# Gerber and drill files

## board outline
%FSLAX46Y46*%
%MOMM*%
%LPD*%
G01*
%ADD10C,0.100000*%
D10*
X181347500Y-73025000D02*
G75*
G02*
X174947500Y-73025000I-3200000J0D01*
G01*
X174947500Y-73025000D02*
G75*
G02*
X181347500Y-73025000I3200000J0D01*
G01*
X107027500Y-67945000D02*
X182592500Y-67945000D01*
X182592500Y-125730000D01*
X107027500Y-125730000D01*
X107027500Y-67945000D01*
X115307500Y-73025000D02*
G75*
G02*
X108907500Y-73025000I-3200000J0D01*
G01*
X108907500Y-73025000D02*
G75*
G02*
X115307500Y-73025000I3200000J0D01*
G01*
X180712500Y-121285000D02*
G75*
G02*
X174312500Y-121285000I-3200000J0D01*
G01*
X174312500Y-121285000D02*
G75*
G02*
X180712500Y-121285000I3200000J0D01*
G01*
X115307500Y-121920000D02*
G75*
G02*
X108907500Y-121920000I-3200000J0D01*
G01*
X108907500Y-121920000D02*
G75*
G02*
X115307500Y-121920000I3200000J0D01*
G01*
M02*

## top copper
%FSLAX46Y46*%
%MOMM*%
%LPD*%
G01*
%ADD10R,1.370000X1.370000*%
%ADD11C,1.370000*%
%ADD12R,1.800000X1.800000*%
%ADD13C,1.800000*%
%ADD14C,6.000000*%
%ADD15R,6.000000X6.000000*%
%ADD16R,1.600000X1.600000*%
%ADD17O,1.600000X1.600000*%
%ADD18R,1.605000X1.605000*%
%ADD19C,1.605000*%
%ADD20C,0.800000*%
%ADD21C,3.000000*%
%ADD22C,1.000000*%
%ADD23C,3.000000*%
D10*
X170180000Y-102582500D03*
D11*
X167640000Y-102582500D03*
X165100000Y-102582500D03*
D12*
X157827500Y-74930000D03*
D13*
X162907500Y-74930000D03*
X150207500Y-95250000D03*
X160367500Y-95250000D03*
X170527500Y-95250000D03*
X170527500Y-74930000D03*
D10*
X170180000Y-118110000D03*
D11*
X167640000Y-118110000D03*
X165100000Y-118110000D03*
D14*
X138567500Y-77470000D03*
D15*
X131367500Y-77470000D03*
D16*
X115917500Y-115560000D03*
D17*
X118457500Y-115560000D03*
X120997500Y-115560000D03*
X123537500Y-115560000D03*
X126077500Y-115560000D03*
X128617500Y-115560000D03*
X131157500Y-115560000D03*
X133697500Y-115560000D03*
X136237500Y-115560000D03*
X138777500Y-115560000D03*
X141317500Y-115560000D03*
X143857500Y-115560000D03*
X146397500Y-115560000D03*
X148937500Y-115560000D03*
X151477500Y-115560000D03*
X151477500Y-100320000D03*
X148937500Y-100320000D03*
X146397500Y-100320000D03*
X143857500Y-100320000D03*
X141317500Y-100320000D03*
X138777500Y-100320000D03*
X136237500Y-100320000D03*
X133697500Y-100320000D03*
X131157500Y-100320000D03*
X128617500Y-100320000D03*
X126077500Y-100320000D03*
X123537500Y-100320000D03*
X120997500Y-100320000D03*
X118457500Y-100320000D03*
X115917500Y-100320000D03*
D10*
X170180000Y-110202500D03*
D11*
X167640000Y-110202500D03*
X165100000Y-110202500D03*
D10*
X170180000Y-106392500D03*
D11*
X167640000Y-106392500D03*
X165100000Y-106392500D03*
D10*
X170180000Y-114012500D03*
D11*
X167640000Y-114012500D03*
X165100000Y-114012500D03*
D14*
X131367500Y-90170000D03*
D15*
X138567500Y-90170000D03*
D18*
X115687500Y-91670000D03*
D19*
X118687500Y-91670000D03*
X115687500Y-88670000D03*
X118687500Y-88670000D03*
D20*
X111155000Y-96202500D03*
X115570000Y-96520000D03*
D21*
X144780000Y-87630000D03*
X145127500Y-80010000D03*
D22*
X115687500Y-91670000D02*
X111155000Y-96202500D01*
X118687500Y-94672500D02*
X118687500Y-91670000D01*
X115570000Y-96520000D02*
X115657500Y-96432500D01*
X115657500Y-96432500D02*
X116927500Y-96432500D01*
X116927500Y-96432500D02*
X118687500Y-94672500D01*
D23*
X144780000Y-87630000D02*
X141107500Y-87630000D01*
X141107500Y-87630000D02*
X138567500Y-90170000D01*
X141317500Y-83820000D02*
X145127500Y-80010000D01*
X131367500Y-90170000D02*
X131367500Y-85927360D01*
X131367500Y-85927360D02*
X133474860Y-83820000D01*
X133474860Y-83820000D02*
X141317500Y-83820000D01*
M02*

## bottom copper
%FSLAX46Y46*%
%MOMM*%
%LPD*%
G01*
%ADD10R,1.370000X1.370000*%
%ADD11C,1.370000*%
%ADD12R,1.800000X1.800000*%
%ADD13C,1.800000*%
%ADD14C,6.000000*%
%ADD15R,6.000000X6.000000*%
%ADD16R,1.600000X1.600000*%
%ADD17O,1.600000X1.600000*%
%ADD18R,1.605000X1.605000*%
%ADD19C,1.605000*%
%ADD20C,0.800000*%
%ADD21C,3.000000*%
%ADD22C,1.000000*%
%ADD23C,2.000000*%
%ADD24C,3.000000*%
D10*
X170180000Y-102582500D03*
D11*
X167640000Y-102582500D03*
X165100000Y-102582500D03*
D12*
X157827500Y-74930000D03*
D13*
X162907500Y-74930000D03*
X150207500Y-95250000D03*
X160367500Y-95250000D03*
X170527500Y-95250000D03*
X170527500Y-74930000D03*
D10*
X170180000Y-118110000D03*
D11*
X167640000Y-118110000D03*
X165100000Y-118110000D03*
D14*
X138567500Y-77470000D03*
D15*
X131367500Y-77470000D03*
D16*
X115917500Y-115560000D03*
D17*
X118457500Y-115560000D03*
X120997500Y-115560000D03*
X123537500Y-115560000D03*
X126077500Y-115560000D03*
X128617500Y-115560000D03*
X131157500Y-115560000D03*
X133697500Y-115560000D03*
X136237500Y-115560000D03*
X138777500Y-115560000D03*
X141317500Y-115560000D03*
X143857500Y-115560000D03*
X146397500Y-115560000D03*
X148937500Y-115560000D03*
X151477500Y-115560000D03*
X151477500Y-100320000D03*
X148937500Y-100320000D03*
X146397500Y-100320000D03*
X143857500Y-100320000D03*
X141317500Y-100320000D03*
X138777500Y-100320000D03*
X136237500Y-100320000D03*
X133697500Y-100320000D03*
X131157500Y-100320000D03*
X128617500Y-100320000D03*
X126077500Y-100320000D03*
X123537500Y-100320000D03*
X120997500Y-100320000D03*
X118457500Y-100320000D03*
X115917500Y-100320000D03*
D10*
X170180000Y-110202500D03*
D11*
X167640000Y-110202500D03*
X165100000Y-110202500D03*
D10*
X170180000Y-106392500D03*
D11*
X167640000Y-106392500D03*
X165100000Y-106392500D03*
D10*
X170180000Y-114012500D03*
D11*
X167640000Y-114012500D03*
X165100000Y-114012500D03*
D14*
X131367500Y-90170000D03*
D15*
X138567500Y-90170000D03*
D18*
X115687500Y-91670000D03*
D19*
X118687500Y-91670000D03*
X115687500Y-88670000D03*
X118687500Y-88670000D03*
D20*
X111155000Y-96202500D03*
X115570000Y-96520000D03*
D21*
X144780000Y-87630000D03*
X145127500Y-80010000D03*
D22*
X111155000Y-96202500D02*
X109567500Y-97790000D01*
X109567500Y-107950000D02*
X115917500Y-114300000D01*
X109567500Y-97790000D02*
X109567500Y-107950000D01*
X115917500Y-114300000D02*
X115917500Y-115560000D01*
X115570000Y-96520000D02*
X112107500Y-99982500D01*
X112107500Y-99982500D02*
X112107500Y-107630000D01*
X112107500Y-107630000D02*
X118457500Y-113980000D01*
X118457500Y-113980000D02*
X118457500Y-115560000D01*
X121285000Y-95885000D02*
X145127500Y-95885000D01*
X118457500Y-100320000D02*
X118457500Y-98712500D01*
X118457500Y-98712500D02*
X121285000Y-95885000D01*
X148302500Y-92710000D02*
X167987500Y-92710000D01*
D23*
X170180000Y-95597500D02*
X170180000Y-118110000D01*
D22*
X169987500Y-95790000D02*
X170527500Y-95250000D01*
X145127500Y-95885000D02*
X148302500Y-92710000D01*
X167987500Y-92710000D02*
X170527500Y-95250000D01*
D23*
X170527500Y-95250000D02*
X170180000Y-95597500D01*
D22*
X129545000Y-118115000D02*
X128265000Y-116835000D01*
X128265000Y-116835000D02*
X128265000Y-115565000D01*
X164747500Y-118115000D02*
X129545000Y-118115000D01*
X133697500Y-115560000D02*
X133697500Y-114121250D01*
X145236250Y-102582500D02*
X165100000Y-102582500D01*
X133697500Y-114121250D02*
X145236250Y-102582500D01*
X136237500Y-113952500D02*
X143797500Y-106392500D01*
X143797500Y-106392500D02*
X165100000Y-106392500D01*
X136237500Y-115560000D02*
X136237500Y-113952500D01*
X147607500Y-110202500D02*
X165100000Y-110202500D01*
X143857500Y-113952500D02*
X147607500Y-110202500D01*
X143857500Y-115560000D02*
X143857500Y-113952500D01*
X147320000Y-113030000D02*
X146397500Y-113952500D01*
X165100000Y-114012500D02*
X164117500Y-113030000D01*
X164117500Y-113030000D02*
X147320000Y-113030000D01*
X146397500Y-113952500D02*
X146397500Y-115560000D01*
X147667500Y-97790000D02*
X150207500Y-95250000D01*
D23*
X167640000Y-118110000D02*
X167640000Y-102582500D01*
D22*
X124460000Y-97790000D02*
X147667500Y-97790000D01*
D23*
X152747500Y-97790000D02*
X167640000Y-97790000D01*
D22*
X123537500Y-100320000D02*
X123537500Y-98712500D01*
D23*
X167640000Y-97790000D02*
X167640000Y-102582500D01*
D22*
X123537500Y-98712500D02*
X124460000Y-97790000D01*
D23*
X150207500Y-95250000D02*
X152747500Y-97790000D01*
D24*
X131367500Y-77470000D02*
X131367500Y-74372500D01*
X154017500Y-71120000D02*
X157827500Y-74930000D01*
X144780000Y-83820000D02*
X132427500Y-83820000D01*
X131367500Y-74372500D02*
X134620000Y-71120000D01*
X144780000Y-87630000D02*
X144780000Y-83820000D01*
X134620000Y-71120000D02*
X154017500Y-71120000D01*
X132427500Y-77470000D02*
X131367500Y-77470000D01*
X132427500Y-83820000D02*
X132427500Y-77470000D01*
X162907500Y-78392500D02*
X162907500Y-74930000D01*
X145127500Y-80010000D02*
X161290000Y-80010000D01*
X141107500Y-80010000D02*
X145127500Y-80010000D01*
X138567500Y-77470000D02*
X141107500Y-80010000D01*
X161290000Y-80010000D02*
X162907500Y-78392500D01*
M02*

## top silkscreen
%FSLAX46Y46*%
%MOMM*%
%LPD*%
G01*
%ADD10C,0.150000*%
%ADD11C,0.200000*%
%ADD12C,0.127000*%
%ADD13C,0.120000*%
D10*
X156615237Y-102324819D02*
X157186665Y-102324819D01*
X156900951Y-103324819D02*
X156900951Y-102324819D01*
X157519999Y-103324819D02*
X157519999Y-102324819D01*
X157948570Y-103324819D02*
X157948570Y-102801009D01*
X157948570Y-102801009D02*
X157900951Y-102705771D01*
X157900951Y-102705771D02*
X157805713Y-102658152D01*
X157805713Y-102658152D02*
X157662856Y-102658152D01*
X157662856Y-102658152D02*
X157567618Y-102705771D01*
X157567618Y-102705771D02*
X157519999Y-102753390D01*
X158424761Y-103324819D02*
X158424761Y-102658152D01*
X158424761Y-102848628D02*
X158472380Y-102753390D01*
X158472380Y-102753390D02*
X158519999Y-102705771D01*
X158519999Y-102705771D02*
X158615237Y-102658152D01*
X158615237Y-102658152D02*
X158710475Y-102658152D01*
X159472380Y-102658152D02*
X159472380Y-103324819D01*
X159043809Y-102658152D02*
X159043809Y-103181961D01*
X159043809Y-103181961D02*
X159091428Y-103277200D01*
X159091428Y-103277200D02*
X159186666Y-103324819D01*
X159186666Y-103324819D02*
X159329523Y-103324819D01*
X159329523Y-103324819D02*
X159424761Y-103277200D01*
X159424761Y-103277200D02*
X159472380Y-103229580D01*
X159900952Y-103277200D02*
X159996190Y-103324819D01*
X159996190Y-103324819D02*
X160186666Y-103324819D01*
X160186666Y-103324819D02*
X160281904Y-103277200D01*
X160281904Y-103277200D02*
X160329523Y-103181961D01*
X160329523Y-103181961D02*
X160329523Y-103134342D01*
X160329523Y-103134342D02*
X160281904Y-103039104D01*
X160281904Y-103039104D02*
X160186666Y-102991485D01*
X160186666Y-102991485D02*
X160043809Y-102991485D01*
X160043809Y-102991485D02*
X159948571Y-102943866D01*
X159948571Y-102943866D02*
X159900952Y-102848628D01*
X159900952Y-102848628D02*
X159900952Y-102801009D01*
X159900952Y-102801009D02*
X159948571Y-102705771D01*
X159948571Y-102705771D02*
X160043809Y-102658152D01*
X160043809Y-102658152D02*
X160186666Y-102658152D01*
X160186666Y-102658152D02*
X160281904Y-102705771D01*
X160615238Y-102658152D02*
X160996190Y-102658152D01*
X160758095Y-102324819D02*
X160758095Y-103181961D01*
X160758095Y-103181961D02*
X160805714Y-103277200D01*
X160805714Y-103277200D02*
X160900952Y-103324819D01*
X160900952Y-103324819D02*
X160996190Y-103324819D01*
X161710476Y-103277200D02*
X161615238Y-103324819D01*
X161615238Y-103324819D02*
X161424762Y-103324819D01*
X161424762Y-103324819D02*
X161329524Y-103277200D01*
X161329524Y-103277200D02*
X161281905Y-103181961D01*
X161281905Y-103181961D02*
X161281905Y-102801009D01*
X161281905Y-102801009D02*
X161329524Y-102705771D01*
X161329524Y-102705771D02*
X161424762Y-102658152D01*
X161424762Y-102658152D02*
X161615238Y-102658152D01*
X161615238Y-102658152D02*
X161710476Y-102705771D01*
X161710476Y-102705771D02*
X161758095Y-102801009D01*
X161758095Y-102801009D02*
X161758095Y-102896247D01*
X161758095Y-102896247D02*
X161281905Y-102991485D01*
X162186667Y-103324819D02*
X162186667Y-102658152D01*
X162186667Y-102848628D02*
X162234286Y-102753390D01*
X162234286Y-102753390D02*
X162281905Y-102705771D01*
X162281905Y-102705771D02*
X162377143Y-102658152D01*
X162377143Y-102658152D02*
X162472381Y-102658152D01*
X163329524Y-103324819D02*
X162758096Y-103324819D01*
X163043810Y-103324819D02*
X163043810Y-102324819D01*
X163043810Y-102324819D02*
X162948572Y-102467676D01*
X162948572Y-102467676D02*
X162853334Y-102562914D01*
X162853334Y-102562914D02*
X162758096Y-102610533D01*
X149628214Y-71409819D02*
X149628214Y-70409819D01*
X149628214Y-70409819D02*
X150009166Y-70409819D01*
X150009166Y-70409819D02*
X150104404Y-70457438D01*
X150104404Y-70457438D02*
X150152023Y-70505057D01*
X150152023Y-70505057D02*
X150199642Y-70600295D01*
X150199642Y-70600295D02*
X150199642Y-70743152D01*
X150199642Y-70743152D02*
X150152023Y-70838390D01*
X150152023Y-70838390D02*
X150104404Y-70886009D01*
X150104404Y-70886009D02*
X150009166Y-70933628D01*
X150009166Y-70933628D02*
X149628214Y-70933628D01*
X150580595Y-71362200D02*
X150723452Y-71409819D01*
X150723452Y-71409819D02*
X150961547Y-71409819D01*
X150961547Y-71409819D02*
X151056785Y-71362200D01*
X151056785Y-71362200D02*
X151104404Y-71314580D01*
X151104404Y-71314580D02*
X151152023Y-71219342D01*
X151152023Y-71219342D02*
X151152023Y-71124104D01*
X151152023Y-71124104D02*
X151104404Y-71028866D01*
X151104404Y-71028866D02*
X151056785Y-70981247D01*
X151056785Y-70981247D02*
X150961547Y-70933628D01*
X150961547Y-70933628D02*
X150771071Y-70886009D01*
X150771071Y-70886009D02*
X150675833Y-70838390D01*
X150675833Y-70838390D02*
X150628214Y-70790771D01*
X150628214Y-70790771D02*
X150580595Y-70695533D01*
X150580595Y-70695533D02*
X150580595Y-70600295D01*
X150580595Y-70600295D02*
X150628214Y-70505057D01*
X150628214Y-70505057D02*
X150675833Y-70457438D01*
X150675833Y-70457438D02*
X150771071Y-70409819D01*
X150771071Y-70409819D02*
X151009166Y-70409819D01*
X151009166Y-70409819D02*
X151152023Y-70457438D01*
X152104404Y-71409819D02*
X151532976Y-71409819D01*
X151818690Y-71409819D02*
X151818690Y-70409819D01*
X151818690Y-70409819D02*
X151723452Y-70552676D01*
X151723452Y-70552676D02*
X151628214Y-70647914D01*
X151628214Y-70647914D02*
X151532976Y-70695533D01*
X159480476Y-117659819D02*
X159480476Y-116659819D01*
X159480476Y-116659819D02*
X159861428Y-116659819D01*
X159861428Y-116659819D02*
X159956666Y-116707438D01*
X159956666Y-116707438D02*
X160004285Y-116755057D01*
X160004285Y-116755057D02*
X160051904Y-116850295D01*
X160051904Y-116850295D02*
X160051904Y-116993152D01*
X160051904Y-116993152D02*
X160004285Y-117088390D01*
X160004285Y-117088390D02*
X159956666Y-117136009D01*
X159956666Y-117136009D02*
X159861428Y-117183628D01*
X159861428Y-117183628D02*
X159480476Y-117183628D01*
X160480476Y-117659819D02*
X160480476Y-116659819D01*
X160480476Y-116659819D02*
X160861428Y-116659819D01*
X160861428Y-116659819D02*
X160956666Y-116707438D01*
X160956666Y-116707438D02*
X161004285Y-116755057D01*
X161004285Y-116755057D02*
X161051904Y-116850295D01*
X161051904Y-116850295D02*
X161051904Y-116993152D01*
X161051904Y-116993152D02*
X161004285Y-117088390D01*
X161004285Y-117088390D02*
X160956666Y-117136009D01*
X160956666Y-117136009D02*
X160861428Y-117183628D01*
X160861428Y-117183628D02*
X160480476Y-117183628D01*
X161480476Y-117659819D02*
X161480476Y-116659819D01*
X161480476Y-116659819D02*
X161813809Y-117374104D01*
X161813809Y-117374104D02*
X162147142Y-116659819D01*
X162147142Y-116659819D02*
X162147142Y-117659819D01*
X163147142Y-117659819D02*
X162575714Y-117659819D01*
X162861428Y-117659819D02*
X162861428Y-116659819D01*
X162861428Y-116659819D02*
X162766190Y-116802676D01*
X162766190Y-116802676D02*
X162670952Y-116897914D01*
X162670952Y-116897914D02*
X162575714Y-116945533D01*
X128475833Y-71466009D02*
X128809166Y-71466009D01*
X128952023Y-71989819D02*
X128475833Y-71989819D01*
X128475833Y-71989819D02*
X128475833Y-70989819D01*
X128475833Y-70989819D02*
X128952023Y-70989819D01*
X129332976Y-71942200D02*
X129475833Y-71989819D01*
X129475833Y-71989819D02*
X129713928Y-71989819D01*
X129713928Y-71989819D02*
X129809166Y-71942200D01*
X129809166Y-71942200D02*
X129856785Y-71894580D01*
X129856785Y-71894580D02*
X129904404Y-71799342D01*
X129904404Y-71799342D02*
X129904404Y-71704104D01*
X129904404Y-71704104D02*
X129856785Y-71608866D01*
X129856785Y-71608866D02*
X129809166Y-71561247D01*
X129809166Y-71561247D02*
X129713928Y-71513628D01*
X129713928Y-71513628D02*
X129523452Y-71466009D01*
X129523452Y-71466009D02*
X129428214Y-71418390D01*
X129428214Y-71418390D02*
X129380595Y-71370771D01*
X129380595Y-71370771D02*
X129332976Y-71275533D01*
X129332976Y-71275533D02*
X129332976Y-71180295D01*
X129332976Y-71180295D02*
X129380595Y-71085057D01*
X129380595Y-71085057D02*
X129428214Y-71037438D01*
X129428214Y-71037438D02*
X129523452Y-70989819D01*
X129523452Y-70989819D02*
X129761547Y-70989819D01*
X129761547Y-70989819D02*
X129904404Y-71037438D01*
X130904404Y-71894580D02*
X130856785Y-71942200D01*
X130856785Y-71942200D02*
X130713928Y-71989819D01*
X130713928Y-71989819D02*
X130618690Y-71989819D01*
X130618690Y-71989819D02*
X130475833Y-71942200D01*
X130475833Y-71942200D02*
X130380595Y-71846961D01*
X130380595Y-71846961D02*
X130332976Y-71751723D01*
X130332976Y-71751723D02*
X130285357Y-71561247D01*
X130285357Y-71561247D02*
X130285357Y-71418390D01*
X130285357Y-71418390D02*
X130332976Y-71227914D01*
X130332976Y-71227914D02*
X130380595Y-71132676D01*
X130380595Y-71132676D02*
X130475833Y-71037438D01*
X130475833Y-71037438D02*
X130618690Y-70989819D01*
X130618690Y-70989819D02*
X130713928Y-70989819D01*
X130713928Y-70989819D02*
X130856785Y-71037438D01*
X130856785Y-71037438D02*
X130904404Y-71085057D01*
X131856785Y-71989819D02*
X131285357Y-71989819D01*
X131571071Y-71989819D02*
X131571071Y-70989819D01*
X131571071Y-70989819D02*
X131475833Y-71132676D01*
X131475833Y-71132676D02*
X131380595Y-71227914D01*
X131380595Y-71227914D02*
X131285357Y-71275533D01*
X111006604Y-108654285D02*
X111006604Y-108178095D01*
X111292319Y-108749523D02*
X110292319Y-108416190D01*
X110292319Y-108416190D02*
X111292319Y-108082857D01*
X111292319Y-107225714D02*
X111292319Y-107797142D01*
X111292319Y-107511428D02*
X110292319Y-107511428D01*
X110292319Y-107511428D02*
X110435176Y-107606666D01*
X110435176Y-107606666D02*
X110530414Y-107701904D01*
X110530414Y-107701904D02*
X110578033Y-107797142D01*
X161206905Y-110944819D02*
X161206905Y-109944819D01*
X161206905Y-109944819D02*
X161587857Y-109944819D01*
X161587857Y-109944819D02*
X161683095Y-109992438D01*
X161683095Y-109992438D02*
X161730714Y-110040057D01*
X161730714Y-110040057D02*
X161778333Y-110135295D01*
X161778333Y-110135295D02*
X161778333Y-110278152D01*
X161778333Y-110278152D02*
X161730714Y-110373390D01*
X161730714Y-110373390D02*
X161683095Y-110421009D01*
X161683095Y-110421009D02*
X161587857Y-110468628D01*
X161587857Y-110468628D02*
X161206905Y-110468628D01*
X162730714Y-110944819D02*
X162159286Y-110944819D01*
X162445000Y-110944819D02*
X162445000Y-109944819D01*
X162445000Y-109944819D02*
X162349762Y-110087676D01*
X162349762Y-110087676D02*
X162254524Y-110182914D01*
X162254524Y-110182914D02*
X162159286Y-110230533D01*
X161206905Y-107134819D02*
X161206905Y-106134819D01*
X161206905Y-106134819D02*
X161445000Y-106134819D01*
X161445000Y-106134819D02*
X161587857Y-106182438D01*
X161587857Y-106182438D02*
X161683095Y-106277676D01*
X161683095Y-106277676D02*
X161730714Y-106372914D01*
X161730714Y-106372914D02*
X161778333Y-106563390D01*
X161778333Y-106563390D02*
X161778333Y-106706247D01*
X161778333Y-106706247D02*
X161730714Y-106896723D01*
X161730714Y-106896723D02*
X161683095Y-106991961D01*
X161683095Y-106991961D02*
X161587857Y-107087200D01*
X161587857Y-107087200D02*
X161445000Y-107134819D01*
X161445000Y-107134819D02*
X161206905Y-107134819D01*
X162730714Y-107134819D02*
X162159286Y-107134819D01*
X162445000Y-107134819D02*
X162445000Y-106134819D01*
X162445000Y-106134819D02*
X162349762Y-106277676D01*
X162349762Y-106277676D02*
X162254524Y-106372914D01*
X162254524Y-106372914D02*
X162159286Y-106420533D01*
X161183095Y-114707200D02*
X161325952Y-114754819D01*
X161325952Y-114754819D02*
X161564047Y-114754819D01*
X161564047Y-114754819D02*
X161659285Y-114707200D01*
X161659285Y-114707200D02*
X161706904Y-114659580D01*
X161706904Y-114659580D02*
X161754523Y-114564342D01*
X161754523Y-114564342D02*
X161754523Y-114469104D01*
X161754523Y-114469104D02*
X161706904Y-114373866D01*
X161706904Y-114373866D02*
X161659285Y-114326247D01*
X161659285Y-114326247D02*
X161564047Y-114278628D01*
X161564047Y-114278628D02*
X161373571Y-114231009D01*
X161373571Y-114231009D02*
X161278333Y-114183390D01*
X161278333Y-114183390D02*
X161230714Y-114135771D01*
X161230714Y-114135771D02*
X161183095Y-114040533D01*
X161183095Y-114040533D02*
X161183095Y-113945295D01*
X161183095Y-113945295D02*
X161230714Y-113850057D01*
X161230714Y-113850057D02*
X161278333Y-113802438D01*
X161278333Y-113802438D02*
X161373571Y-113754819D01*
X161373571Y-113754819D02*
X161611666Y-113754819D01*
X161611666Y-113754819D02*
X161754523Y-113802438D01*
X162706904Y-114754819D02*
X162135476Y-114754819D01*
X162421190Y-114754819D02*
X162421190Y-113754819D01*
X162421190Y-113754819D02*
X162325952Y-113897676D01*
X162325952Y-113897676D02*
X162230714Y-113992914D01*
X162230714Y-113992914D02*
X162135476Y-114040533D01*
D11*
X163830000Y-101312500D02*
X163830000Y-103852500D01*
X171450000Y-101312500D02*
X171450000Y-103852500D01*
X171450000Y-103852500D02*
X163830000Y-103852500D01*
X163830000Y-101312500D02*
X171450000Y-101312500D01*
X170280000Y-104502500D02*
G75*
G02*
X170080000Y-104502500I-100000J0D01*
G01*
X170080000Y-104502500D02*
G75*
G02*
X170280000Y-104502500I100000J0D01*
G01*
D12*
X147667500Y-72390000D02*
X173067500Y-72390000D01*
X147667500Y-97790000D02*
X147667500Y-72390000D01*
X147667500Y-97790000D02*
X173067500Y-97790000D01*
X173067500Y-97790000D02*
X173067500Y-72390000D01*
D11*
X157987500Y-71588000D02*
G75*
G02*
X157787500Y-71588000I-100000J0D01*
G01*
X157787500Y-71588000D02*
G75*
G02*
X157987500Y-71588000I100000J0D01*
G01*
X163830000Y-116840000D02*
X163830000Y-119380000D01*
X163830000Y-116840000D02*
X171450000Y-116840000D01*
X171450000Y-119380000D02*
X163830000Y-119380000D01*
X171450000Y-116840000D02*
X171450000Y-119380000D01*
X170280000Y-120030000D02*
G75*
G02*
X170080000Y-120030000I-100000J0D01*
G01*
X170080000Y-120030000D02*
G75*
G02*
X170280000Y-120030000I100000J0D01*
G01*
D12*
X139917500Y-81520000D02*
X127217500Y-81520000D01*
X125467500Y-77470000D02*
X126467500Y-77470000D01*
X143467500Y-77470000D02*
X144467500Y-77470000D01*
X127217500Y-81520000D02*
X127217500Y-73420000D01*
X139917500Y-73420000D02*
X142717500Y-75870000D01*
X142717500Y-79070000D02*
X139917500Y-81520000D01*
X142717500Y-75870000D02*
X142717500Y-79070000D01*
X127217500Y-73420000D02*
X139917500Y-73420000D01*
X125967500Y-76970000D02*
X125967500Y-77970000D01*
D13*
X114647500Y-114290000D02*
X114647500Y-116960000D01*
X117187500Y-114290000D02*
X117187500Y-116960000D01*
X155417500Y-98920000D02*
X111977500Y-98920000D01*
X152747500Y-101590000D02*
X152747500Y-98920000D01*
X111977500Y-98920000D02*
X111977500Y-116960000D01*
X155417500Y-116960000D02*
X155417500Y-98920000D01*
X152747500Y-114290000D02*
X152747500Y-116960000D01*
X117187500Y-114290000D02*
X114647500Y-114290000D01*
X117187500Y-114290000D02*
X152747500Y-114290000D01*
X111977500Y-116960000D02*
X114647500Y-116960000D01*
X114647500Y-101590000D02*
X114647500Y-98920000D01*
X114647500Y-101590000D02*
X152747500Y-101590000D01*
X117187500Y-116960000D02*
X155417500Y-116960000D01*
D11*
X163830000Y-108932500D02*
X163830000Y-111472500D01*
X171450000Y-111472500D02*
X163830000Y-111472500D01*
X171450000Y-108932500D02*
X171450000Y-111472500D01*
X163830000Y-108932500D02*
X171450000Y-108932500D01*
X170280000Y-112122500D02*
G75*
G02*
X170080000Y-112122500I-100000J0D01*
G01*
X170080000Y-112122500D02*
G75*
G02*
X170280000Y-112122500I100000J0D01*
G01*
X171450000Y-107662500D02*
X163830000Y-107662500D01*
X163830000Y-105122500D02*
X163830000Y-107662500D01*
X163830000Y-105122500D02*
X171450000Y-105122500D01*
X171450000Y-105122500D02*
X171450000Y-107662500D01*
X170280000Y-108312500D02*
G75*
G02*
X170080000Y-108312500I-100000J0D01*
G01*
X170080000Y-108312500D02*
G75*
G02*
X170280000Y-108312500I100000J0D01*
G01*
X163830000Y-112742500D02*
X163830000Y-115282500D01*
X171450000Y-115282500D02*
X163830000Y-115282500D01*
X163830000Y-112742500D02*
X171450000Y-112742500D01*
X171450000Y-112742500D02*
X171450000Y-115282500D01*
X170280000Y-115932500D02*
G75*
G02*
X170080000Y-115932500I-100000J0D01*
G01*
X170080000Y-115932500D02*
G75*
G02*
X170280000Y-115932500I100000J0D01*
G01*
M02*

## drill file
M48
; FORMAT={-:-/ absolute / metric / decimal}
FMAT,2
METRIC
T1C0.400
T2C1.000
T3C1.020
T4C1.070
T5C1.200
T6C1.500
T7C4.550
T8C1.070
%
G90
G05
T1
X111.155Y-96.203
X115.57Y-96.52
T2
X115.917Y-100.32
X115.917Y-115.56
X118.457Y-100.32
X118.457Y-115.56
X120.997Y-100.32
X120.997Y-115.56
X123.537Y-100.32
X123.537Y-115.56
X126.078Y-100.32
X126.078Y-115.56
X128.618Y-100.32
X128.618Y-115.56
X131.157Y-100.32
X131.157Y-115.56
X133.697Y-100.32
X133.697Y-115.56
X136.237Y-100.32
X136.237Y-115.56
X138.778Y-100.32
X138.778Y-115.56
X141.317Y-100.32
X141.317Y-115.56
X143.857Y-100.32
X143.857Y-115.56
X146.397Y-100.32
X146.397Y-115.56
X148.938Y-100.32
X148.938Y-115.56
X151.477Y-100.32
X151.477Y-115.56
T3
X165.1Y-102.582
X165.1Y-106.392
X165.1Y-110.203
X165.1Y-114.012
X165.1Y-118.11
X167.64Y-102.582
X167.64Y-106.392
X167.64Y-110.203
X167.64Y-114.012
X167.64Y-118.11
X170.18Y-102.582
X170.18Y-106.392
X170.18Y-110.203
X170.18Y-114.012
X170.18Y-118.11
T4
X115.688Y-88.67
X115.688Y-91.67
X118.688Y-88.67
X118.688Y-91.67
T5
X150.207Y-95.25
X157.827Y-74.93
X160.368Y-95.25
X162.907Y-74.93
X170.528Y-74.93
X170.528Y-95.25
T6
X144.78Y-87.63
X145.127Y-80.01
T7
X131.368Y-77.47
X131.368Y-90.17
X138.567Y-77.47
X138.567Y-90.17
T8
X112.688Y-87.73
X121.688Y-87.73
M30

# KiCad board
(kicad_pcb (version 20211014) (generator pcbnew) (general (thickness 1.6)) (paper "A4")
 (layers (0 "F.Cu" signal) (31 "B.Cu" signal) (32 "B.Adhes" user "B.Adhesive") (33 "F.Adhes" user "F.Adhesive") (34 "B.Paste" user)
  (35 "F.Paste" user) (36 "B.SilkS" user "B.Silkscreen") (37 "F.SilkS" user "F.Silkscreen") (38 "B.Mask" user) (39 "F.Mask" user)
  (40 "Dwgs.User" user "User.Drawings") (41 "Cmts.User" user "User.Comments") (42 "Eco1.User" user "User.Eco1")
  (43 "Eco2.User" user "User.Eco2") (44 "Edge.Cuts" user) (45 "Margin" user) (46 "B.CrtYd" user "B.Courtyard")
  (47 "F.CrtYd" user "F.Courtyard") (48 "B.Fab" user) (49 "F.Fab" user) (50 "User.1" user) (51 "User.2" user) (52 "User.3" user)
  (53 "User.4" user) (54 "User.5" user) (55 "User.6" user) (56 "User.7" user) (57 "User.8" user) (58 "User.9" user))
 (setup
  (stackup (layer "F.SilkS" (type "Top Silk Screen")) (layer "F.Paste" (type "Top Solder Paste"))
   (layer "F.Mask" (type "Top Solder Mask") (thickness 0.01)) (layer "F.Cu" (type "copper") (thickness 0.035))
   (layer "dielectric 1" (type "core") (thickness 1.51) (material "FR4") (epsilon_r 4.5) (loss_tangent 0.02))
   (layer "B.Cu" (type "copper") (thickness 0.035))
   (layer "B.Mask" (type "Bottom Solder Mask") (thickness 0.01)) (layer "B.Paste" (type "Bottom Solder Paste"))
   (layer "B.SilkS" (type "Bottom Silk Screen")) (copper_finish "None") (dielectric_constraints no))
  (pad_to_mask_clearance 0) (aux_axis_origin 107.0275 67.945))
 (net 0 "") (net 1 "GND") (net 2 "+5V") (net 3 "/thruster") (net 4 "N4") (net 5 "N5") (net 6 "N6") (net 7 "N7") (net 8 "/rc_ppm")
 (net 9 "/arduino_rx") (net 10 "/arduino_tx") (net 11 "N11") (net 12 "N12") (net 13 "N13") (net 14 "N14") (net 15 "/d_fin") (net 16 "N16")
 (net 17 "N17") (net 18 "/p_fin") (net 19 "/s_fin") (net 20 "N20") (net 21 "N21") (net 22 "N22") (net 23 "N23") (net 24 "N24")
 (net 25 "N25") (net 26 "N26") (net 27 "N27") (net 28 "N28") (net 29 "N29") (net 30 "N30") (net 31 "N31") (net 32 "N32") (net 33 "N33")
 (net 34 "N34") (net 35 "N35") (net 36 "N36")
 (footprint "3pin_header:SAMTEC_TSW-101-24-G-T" (layer "F.Cu") (at 170.18 102.5825 90)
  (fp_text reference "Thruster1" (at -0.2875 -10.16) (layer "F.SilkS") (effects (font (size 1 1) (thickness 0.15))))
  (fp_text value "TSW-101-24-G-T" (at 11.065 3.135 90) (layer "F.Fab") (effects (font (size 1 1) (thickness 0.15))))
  (fp_line (start 1.27 -6.35) (end -1.27 -6.35) (layer "F.SilkS") (width 0.2))
  (fp_line (start 1.27 1.27) (end -1.27 1.27) (layer "F.SilkS") (width 0.2))
  (fp_line (start -1.27 1.27) (end -1.27 -6.35) (layer "F.SilkS") (width 0.2))
  (fp_line (start 1.27 -6.35) (end 1.27 1.27) (layer "F.SilkS") (width 0.2))
  (fp_circle (center -1.92 0) (end -1.82 0) (layer "F.SilkS") (width 0.2) (fill none))
  (pad "01" thru_hole rect locked (at 0 0 90) (size 1.37 1.37) (drill 1.02) (layers *.Cu *.Mask) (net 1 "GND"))
  (pad "02" thru_hole circle locked (at 0 -2.54 90) (size 1.37 1.37) (drill 1.02) (layers *.Cu *.Mask) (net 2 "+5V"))
  (pad "03" thru_hole circle locked (at 0 -5.08 90) (size 1.37 1.37) (drill 1.02) (layers *.Cu *.Mask) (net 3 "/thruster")))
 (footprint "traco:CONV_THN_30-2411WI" (layer "F.Cu") (at 160.3675 85.09)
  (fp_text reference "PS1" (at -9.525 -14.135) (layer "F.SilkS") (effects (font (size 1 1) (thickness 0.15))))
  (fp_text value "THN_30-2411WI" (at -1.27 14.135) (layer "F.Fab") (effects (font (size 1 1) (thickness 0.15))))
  (fp_line (start -12.7 -12.7) (end 12.7 -12.7) (layer "F.SilkS") (width 0.127))
  (fp_line (start -12.7 12.7) (end -12.7 -12.7) (layer "F.SilkS") (width 0.127))
  (fp_line (start -12.7 12.7) (end 12.7 12.7) (layer "F.SilkS") (width 0.127))
  (fp_line (start 12.7 12.7) (end 12.7 -12.7) (layer "F.SilkS") (width 0.127))
  (fp_circle (center -2.48 -13.502) (end -2.38 -13.502) (layer "F.SilkS") (width 0.2) (fill none))
  (pad "1" thru_hole rect locked (at -2.54 -10.16) (size 1.8 1.8) (drill 1.2) (layers *.Cu *.Mask) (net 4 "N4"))
  (pad "2" thru_hole circle locked (at 2.54 -10.16) (size 1.8 1.8) (drill 1.2) (layers *.Cu *.Mask) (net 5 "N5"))
  (pad "3" thru_hole circle locked (at -10.16 10.16) (size 1.8 1.8) (drill 1.2) (layers *.Cu *.Mask) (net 2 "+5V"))
  (pad "4" thru_hole circle locked (at 0 10.16) (size 1.8 1.8) (drill 1.2) (layers *.Cu *.Mask) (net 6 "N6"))
  (pad "5" thru_hole circle locked (at 10.16 10.16) (size 1.8 1.8) (drill 1.2) (layers *.Cu *.Mask) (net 1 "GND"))
  (pad "6" thru_hole circle locked (at 10.16 -10.16) (size 1.8 1.8) (drill 1.2) (layers *.Cu *.Mask) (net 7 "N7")))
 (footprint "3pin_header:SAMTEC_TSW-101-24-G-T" (layer "F.Cu") (at 170.18 118.11 90)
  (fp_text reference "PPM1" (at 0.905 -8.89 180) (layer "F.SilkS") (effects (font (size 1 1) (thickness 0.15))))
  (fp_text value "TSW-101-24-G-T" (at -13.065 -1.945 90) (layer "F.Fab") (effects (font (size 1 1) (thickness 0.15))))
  (fp_line (start 1.27 -6.35) (end -1.27 -6.35) (layer "F.SilkS") (width 0.2))
  (fp_line (start 1.27 -6.35) (end 1.27 1.27) (layer "F.SilkS") (width 0.2))
  (fp_line (start -1.27 1.27) (end -1.27 -6.35) (layer "F.SilkS") (width 0.2))
  (fp_line (start 1.27 1.27) (end -1.27 1.27) (layer "F.SilkS") (width 0.2))
  (fp_circle (center -1.92 0) (end -1.82 0) (layer "F.SilkS") (width 0.2) (fill none))
  (pad "01" thru_hole rect locked (at 0 0 90) (size 1.37 1.37) (drill 1.02) (layers *.Cu *.Mask) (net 1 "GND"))
  (pad "02" thru_hole circle locked (at 0 -2.54 90) (size 1.37 1.37) (drill 1.02) (layers *.Cu *.Mask) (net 2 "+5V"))
  (pad "03" thru_hole circle locked (at 0 -5.08 90) (size 1.37 1.37) (drill 1.02) (layers *.Cu *.Mask) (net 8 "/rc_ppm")))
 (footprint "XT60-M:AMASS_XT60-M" (layer "F.Cu") (at 134.9675 77.47)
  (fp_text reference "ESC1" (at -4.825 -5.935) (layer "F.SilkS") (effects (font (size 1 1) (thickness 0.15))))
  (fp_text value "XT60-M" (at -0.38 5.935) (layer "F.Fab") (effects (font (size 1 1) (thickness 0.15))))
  (fp_line (start 4.95 4.05) (end -7.75 4.05) (layer "F.SilkS") (width 0.127))
  (fp_line (start -9.5 0) (end -8.5 0) (layer "F.SilkS") (width 0.127))
  (fp_line (start 8.5 0) (end 9.5 0) (layer "F.SilkS") (width 0.127))
  (fp_line (start -7.75 4.05) (end -7.75 -4.05) (layer "F.SilkS") (width 0.127))
  (fp_line (start 4.95 -4.05) (end 7.75 -1.6) (layer "F.SilkS") (width 0.127))
  (fp_line (start 7.75 1.6) (end 4.95 4.05) (layer "F.SilkS") (width 0.127))
  (fp_line (start 7.75 -1.6) (end 7.75 1.6) (layer "F.SilkS") (width 0.127))
  (fp_line (start -7.75 -4.05) (end 4.95 -4.05) (layer "F.SilkS") (width 0.127))
  (fp_line (start -9 -0.5) (end -9 0.5) (layer "F.SilkS") (width 0.127))
  (pad "N" thru_hole circle locked (at 3.6 0) (size 6 6) (drill 4.55) (layers *.Cu *.Mask) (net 5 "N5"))
  (pad "P" thru_hole rect locked (at -3.6 0) (size 6 6) (drill 4.55) (layers *.Cu *.Mask) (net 4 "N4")))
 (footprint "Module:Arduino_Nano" (layer "F.Cu") (at 115.9175 115.56 90)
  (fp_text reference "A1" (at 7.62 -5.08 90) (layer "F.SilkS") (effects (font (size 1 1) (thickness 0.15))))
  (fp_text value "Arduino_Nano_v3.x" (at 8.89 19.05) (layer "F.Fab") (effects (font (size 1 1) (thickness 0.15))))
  (fp_line (start 1.27 -1.27) (end -1.4 -1.27) (layer "F.SilkS") (width 0.12))
  (fp_line (start 1.27 1.27) (end -1.4 1.27) (layer "F.SilkS") (width 0.12))
  (fp_line (start 16.64 39.5) (end 16.64 -3.94) (layer "F.SilkS") (width 0.12))
  (fp_line (start 13.97 36.83) (end 16.64 36.83) (layer "F.SilkS") (width 0.12))
  (fp_line (start 16.64 -3.94) (end -1.4 -3.94) (layer "F.SilkS") (width 0.12))
  (fp_line (start -1.4 39.5) (end 16.64 39.5) (layer "F.SilkS") (width 0.12))
  (fp_line (start 1.27 36.83) (end -1.4 36.83) (layer "F.SilkS") (width 0.12))
  (fp_line (start 1.27 1.27) (end 1.27 -1.27) (layer "F.SilkS") (width 0.12))
  (fp_line (start 1.27 1.27) (end 1.27 36.83) (layer "F.SilkS") (width 0.12))
  (fp_line (start -1.4 -3.94) (end -1.4 -1.27) (layer "F.SilkS") (width 0.12))
  (fp_line (start 13.97 -1.27) (end 16.64 -1.27) (layer "F.SilkS") (width 0.12))
  (fp_line (start 13.97 -1.27) (end 13.97 36.83) (layer "F.SilkS") (width 0.12))
  (fp_line (start -1.4 1.27) (end -1.4 39.5) (layer "F.SilkS") (width 0.12))
  (pad "1" thru_hole rect (at 0 0 90) (size 1.6 1.6) (drill 1) (layers *.Cu *.Mask) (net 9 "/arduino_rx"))
  (pad "2" thru_hole oval (at 0 2.54 90) (size 1.6 1.6) (drill 1) (layers *.Cu *.Mask) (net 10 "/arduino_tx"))
  (pad "3" thru_hole oval (at 0 5.08 90) (size 1.6 1.6) (drill 1) (layers *.Cu *.Mask) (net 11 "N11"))
  (pad "4" thru_hole oval (at 0 7.62 90) (size 1.6 1.6) (drill 1) (layers *.Cu *.Mask) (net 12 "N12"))
  (pad "5" thru_hole oval (at 0 10.16 90) (size 1.6 1.6) (drill 1) (layers *.Cu *.Mask) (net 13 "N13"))
  (pad "6" thru_hole oval (at 0 12.7 90) (size 1.6 1.6) (drill 1) (layers *.Cu *.Mask) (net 8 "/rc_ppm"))
  (pad "7" thru_hole oval (at 0 15.24 90) (size 1.6 1.6) (drill 1) (layers *.Cu *.Mask) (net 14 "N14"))
  (pad "8" thru_hole oval (at 0 17.78 90) (size 1.6 1.6) (drill 1) (layers *.Cu *.Mask) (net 3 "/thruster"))
  (pad "9" thru_hole oval (at 0 20.32 90) (size 1.6 1.6) (drill 1) (layers *.Cu *.Mask) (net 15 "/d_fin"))
  (pad "10" thru_hole oval (at 0 22.86 90) (size 1.6 1.6) (drill 1) (layers *.Cu *.Mask) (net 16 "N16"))
  (pad "11" thru_hole oval (at 0 25.4 90) (size 1.6 1.6) (drill 1) (layers *.Cu *.Mask) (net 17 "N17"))
  (pad "12" thru_hole oval (at 0 27.94 90) (size 1.6 1.6) (drill 1) (layers *.Cu *.Mask) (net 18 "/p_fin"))
  (pad "13" thru_hole oval (at 0 30.48 90) (size 1.6 1.6) (drill 1) (layers *.Cu *.Mask) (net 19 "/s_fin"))
  (pad "14" thru_hole oval (at 0 33.02 90) (size 1.6 1.6) (drill 1) (layers *.Cu *.Mask) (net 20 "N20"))
  (pad "15" thru_hole oval (at 0 35.56 90) (size 1.6 1.6) (drill 1) (layers *.Cu *.Mask) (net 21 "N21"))
  (pad "16" thru_hole oval (at 15.24 35.56 90) (size 1.6 1.6) (drill 1) (layers *.Cu *.Mask) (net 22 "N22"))
  (pad "17" thru_hole oval (at 15.24 33.02 90) (size 1.6 1.6) (drill 1) (layers *.Cu *.Mask) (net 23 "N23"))
  (pad "18" thru_hole oval (at 15.24 30.48 90) (size 1.6 1.6) (drill 1) (layers *.Cu *.Mask) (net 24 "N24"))
  (pad "19" thru_hole oval (at 15.24 27.94 90) (size 1.6 1.6) (drill 1) (layers *.Cu *.Mask) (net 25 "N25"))
  (pad "20" thru_hole oval (at 15.24 25.4 90) (size 1.6 1.6) (drill 1) (layers *.Cu *.Mask) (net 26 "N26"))
  (pad "21" thru_hole oval (at 15.24 22.86 90) (size 1.6 1.6) (drill 1) (layers *.Cu *.Mask) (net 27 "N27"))
  (pad "22" thru_hole oval (at 15.24 20.32 90) (size 1.6 1.6) (drill 1) (layers *.Cu *.Mask) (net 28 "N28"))
  (pad "23" thru_hole oval (at 15.24 17.78 90) (size 1.6 1.6) (drill 1) (layers *.Cu *.Mask) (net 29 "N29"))
  (pad "24" thru_hole oval (at 15.24 15.24 90) (size 1.6 1.6) (drill 1) (layers *.Cu *.Mask) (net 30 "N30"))
  (pad "25" thru_hole oval (at 15.24 12.7 90) (size 1.6 1.6) (drill 1) (layers *.Cu *.Mask) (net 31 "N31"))
  (pad "26" thru_hole oval (at 15.24 10.16 90) (size 1.6 1.6) (drill 1) (layers *.Cu *.Mask) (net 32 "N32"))
  (pad "27" thru_hole oval (at 15.24 7.62 90) (size 1.6 1.6) (drill 1) (layers *.Cu *.Mask) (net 2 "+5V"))
  (pad "28" thru_hole oval (at 15.24 5.08 90) (size 1.6 1.6) (drill 1) (layers *.Cu *.Mask) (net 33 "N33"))
  (pad "29" thru_hole oval (at 15.24 2.54 90) (size 1.6 1.6) (drill 1) (layers *.Cu *.Mask) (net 1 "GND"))
  (pad "30" thru_hole oval (at 15.24 0 90) (size 1.6 1.6) (drill 1) (layers *.Cu *.Mask) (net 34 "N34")))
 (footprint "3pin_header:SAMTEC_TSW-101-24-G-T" (layer "F.Cu") (at 170.18 110.2025 90)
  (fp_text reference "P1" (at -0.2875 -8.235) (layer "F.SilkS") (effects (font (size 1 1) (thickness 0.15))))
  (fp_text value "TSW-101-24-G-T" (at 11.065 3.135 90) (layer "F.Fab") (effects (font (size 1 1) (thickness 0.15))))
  (fp_line (start 1.27 -6.35) (end -1.27 -6.35) (layer "F.SilkS") (width 0.2))
  (fp_line (start -1.27 1.27) (end -1.27 -6.35) (layer "F.SilkS") (width 0.2))
  (fp_line (start 1.27 1.27) (end -1.27 1.27) (layer "F.SilkS") (width 0.2))
  (fp_line (start 1.27 -6.35) (end 1.27 1.27) (layer "F.SilkS") (width 0.2))
  (fp_circle (center -1.92 0) (end -1.82 0) (layer "F.SilkS") (width 0.2) (fill none))
  (pad "01" thru_hole rect locked (at 0 0 90) (size 1.37 1.37) (drill 1.02) (layers *.Cu *.Mask) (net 1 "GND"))
  (pad "02" thru_hole circle locked (at 0 -2.54 90) (size 1.37 1.37) (drill 1.02) (layers *.Cu *.Mask) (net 2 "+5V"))
  (pad "03" thru_hole circle locked (at 0 -5.08 90) (size 1.37 1.37) (drill 1.02) (layers *.Cu *.Mask) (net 18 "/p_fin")))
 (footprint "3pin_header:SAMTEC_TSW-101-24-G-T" (layer "F.Cu") (at 170.18 106.3925 90)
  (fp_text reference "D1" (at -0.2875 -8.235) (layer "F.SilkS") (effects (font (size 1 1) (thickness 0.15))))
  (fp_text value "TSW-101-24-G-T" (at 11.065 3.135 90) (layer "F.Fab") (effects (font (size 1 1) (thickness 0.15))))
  (fp_line (start -1.27 1.27) (end -1.27 -6.35) (layer "F.SilkS") (width 0.2))
  (fp_line (start 1.27 -6.35) (end -1.27 -6.35) (layer "F.SilkS") (width 0.2))
  (fp_line (start 1.27 -6.35) (end 1.27 1.27) (layer "F.SilkS") (width 0.2))
  (fp_line (start 1.27 1.27) (end -1.27 1.27) (layer "F.SilkS") (width 0.2))
  (fp_circle (center -1.92 0) (end -1.82 0) (layer "F.SilkS") (width 0.2) (fill none))
  (pad "01" thru_hole rect locked (at 0 0 90) (size 1.37 1.37) (drill 1.02) (layers *.Cu *.Mask) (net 1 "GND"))
  (pad "02" thru_hole circle locked (at 0 -2.54 90) (size 1.37 1.37) (drill 1.02) (layers *.Cu *.Mask) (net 2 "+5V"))
  (pad "03" thru_hole circle locked (at 0 -5.08 90) (size 1.37 1.37) (drill 1.02) (layers *.Cu *.Mask) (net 15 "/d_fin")))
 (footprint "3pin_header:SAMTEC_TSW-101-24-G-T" (layer "F.Cu") (at 170.18 114.0125 90)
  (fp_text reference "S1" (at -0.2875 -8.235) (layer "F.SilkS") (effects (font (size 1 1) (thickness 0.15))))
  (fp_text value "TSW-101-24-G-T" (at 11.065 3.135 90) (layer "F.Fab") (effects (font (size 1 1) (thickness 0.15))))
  (fp_line (start 1.27 -6.35) (end -1.27 -6.35) (layer "F.SilkS") (width 0.2))
  (fp_line (start -1.27 1.27) (end -1.27 -6.35) (layer "F.SilkS") (width 0.2))
  (fp_line (start 1.27 -6.35) (end 1.27 1.27) (layer "F.SilkS") (width 0.2))
  (fp_line (start 1.27 1.27) (end -1.27 1.27) (layer "F.SilkS") (width 0.2))
  (fp_circle (center -1.92 0) (end -1.82 0) (layer "F.SilkS") (width 0.2) (fill none))
  (pad "01" thru_hole rect locked (at 0 0 90) (size 1.37 1.37) (drill 1.02) (layers *.Cu *.Mask) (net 1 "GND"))
  (pad "02" thru_hole circle locked (at 0 -2.54 90) (size 1.37 1.37) (drill 1.02) (layers *.Cu *.Mask) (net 2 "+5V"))
  (pad "03" thru_hole circle locked (at 0 -5.08 90) (size 1.37 1.37) (drill 1.02) (layers *.Cu *.Mask) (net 19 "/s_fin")))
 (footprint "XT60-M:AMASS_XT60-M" (layer "B.Cu") (at 134.9675 90.17 180)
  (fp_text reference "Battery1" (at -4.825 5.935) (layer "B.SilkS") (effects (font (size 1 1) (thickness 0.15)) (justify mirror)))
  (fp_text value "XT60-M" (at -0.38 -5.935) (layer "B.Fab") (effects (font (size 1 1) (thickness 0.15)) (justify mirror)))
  (pad "N" thru_hole circle locked (at 3.6 0 180) (size 6 6) (drill 4.55) (layers *.Cu *.Mask) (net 5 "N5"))
  (pad "P" thru_hole rect locked (at -3.6 0 180) (size 6 6) (drill 4.55) (layers *.Cu *.Mask) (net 4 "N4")))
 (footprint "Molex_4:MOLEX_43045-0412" (layer "B.Cu") (at 117.1875 90.17 180)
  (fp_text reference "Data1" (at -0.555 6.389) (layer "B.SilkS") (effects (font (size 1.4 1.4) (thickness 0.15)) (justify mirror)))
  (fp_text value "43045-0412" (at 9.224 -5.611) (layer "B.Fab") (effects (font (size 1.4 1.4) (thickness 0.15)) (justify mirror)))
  (pad "" np_thru_hole circle locked (at -4.5 2.44 180) (size 1.07 1.07) (drill 1.07) (layers *.Cu *.Mask))
  (pad "" np_thru_hole circle locked (at 4.5 2.44 180) (size 1.07 1.07) (drill 1.07) (layers *.Cu *.Mask))
  (pad "1" thru_hole rect locked (at 1.5 -1.5 180) (size 1.605 1.605) (drill 1.07) (layers *.Cu *.Mask) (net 9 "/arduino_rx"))
  (pad "2" thru_hole circle locked (at -1.5 -1.5 180) (size 1.605 1.605) (drill 1.07) (layers *.Cu *.Mask) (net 10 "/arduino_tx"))
  (pad "3" thru_hole circle locked (at 1.5 1.5 180) (size 1.605 1.605) (drill 1.07) (layers *.Cu *.Mask) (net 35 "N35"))
  (pad "4" thru_hole circle locked (at -1.5 1.5 180) (size 1.605 1.605) (drill 1.07) (layers *.Cu *.Mask) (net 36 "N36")))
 (gr_circle (center 178.1475 73.025) (end 181.3475 73.025) (layer "Edge.Cuts") (width 0.1) (fill none))
 (gr_rect (start 182.5925 125.73) (end 107.0275 67.945) (layer "Edge.Cuts") (width 0.1) (fill none))
 (gr_circle (center 112.1075 73.025) (end 115.3075 73.025) (layer "Edge.Cuts") (width 0.1) (fill none))
 (gr_circle (center 177.5125 121.285) (end 180.7125 121.285) (layer "Edge.Cuts") (width 0.1) (fill none))
 (gr_circle (center 112.1075 121.92) (end 115.3075 121.92) (layer "Edge.Cuts") (width 0.1) (fill none))
 (segment (start 115.6875 91.67) (end 111.155 96.2025) (width 1) (layer "F.Cu") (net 9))
 (via (at 111.155 96.2025) (size 0.8) (drill 0.4) (layers "F.Cu" "B.Cu") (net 9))
 (segment (start 111.155 96.2025) (end 109.5675 97.79) (width 1) (layer "B.Cu") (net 9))
 (segment (start 109.5675 107.95) (end 115.9175 114.3) (width 1) (layer "B.Cu") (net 9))
 (segment (start 109.5675 97.79) (end 109.5675 107.95) (width 1) (layer "B.Cu") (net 9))
 (segment (start 115.9175 114.3) (end 115.9175 115.56) (width 1) (layer "B.Cu") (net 9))
 (segment (start 118.6875 94.6725) (end 118.6875 91.67) (width 1) (layer "F.Cu") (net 10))
 (segment (start 115.57 96.52) (end 115.6575 96.4325) (width 1) (layer "F.Cu") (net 10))
 (segment (start 115.6575 96.4325) (end 116.9275 96.4325) (width 1) (layer "F.Cu") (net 10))
 (segment (start 116.9275 96.4325) (end 118.6875 94.6725) (width 1) (layer "F.Cu") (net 10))
 (via (at 115.57 96.52) (size 0.8) (drill 0.4) (layers "F.Cu" "B.Cu") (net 10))
 (segment (start 115.57 96.52) (end 112.1075 99.9825) (width 1) (layer "B.Cu") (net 10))
 (segment (start 112.1075 99.9825) (end 112.1075 107.63) (width 1) (layer "B.Cu") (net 10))
 (segment (start 112.1075 107.63) (end 118.4575 113.98) (width 1) (layer "B.Cu") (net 10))
 (segment (start 118.4575 113.98) (end 118.4575 115.56) (width 1) (layer "B.Cu") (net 10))
 (segment (start 121.285 95.885) (end 145.1275 95.885) (width 1) (layer "B.Cu") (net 1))
 (segment (start 118.4575 100.32) (end 118.4575 98.7125) (width 1) (layer "B.Cu") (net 1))
 (segment (start 118.4575 98.7125) (end 121.285 95.885) (width 1) (layer "B.Cu") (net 1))
 (segment (start 148.3025 92.71) (end 167.9875 92.71) (width 1) (layer "B.Cu") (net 1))
 (segment (start 170.18 95.5975) (end 170.18 118.11) (width 2) (layer "B.Cu") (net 1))
 (segment (start 169.9875 95.79) (end 170.5275 95.25) (width 1) (layer "B.Cu") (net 1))
 (segment (start 145.1275 95.885) (end 148.3025 92.71) (width 1) (layer "B.Cu") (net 1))
 (segment (start 167.9875 92.71) (end 170.5275 95.25) (width 1) (layer "B.Cu") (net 1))
 (segment (start 170.5275 95.25) (end 170.18 95.5975) (width 2) (layer "B.Cu") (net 1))
 (segment (start 129.545 118.115) (end 128.265 116.835) (width 1) (layer "B.Cu") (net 8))
 (segment (start 128.265 116.835) (end 128.265 115.565) (width 1) (layer "B.Cu") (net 8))
 (segment (start 164.7475 118.115) (end 129.545 118.115) (width 1) (layer "B.Cu") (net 8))
 (segment (start 133.6975 115.56) (end 133.6975 114.12125) (width 1) (layer "B.Cu") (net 3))
 (segment (start 145.23625 102.5825) (end 165.1 102.5825) (width 1) (layer "B.Cu") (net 3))
 (segment (start 133.6975 114.12125) (end 145.23625 102.5825) (width 1) (layer "B.Cu") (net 3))
 (segment (start 136.2375 113.9525) (end 143.7975 106.3925) (width 1) (layer "B.Cu") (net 15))
 (segment (start 143.7975 106.3925) (end 165.1 106.3925) (width 1) (layer "B.Cu") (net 15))
 (segment (start 136.2375 115.56) (end 136.2375 113.9525) (width 1) (layer "B.Cu") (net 15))
 (segment (start 147.6075 110.2025) (end 165.1 110.2025) (width 1) (layer "B.Cu") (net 18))
 (segment (start 143.8575 113.9525) (end 147.6075 110.2025) (width 1) (layer "B.Cu") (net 18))
 (segment (start 143.8575 115.56) (end 143.8575 113.9525) (width 1) (layer "B.Cu") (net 18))
 (segment (start 147.32 113.03) (end 146.3975 113.9525) (width 1) (layer "B.Cu") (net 19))
 (segment (start 165.1 114.0125) (end 164.1175 113.03) (width 1) (layer "B.Cu") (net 19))
 (segment (start 164.1175 113.03) (end 147.32 113.03) (width 1) (layer "B.Cu") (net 19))
 (segment (start 146.3975 113.9525) (end 146.3975 115.56) (width 1) (layer "B.Cu") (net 19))
 (segment (start 147.6675 97.79) (end 150.2075 95.25) (width 1) (layer "B.Cu") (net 2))
 (segment (start 167.64 118.11) (end 167.64 102.5825) (width 2) (layer "B.Cu") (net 2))
 (segment (start 124.46 97.79) (end 147.6675 97.79) (width 1) (layer "B.Cu") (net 2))
 (segment (start 152.7475 97.79) (end 167.64 97.79) (width 2) (layer "B.Cu") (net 2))
 (segment (start 123.5375 100.32) (end 123.5375 98.7125) (width 1) (layer "B.Cu") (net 2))
 (segment (start 167.64 97.79) (end 167.64 102.5825) (width 2) (layer "B.Cu") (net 2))
 (segment (start 123.5375 98.7125) (end 124.46 97.79) (width 1) (layer "B.Cu") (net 2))
 (segment (start 150.2075 95.25) (end 152.7475 97.79) (width 2) (layer "B.Cu") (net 2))
 (segment (start 144.78 87.63) (end 141.1075 87.63) (width 3) (layer "F.Cu") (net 4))
 (segment (start 141.1075 87.63) (end 138.5675 90.17) (width 3) (layer "F.Cu") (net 4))
 (via (at 144.78 87.63) (size 3) (drill 1.5) (layers "F.Cu" "B.Cu") (free) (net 4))
 (segment (start 131.3675 77.47) (end 131.3675 74.3725) (width 3) (layer "B.Cu") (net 4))
 (segment (start 154.0175 71.12) (end 157.8275 74.93) (width 3) (layer "B.Cu") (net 4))
 (segment (start 144.78 83.82) (end 132.4275 83.82) (width 3) (layer "B.Cu") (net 4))
 (segment (start 131.3675 74.3725) (end 134.62 71.12) (width 3) (layer "B.Cu") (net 4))
 (segment (start 144.78 87.63) (end 144.78 83.82) (width 3) (layer "B.Cu") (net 4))
 (segment (start 134.62 71.12) (end 154.0175 71.12) (width 3) (layer "B.Cu") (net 4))
 (segment (start 132.4275 77.47) (end 131.3675 77.47) (width 3) (layer "B.Cu") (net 4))
 (segment (start 132.4275 83.82) (end 132.4275 77.47) (width 3) (layer "B.Cu") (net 4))
 (segment (start 141.3175 83.82) (end 145.1275 80.01) (width 3) (layer "F.Cu") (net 5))
 (segment (start 131.3675 90.17) (end 131.3675 85.92736) (width 3) (layer "F.Cu") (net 5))
 (segment (start 131.3675 85.92736) (end 133.47486 83.82) (width 3) (layer "F.Cu") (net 5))
 (segment (start 133.47486 83.82) (end 141.3175 83.82) (width 3) (layer "F.Cu") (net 5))
 (via (at 145.1275 80.01) (size 3) (drill 1.5) (layers "F.Cu" "B.Cu") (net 5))
 (segment (start 162.9075 78.3925) (end 162.9075 74.93) (width 3) (layer "B.Cu") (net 5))
 (segment (start 145.1275 80.01) (end 161.29 80.01) (width 3) (layer "B.Cu") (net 5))
 (segment (start 141.1075 80.01) (end 145.1275 80.01) (width 3) (layer "B.Cu") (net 5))
 (segment (start 138.5675 77.47) (end 141.1075 80.01) (width 3) (layer "B.Cu") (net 5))
 (segment (start 161.29 80.01) (end 162.9075 78.3925) (width 3) (layer "B.Cu") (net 5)))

